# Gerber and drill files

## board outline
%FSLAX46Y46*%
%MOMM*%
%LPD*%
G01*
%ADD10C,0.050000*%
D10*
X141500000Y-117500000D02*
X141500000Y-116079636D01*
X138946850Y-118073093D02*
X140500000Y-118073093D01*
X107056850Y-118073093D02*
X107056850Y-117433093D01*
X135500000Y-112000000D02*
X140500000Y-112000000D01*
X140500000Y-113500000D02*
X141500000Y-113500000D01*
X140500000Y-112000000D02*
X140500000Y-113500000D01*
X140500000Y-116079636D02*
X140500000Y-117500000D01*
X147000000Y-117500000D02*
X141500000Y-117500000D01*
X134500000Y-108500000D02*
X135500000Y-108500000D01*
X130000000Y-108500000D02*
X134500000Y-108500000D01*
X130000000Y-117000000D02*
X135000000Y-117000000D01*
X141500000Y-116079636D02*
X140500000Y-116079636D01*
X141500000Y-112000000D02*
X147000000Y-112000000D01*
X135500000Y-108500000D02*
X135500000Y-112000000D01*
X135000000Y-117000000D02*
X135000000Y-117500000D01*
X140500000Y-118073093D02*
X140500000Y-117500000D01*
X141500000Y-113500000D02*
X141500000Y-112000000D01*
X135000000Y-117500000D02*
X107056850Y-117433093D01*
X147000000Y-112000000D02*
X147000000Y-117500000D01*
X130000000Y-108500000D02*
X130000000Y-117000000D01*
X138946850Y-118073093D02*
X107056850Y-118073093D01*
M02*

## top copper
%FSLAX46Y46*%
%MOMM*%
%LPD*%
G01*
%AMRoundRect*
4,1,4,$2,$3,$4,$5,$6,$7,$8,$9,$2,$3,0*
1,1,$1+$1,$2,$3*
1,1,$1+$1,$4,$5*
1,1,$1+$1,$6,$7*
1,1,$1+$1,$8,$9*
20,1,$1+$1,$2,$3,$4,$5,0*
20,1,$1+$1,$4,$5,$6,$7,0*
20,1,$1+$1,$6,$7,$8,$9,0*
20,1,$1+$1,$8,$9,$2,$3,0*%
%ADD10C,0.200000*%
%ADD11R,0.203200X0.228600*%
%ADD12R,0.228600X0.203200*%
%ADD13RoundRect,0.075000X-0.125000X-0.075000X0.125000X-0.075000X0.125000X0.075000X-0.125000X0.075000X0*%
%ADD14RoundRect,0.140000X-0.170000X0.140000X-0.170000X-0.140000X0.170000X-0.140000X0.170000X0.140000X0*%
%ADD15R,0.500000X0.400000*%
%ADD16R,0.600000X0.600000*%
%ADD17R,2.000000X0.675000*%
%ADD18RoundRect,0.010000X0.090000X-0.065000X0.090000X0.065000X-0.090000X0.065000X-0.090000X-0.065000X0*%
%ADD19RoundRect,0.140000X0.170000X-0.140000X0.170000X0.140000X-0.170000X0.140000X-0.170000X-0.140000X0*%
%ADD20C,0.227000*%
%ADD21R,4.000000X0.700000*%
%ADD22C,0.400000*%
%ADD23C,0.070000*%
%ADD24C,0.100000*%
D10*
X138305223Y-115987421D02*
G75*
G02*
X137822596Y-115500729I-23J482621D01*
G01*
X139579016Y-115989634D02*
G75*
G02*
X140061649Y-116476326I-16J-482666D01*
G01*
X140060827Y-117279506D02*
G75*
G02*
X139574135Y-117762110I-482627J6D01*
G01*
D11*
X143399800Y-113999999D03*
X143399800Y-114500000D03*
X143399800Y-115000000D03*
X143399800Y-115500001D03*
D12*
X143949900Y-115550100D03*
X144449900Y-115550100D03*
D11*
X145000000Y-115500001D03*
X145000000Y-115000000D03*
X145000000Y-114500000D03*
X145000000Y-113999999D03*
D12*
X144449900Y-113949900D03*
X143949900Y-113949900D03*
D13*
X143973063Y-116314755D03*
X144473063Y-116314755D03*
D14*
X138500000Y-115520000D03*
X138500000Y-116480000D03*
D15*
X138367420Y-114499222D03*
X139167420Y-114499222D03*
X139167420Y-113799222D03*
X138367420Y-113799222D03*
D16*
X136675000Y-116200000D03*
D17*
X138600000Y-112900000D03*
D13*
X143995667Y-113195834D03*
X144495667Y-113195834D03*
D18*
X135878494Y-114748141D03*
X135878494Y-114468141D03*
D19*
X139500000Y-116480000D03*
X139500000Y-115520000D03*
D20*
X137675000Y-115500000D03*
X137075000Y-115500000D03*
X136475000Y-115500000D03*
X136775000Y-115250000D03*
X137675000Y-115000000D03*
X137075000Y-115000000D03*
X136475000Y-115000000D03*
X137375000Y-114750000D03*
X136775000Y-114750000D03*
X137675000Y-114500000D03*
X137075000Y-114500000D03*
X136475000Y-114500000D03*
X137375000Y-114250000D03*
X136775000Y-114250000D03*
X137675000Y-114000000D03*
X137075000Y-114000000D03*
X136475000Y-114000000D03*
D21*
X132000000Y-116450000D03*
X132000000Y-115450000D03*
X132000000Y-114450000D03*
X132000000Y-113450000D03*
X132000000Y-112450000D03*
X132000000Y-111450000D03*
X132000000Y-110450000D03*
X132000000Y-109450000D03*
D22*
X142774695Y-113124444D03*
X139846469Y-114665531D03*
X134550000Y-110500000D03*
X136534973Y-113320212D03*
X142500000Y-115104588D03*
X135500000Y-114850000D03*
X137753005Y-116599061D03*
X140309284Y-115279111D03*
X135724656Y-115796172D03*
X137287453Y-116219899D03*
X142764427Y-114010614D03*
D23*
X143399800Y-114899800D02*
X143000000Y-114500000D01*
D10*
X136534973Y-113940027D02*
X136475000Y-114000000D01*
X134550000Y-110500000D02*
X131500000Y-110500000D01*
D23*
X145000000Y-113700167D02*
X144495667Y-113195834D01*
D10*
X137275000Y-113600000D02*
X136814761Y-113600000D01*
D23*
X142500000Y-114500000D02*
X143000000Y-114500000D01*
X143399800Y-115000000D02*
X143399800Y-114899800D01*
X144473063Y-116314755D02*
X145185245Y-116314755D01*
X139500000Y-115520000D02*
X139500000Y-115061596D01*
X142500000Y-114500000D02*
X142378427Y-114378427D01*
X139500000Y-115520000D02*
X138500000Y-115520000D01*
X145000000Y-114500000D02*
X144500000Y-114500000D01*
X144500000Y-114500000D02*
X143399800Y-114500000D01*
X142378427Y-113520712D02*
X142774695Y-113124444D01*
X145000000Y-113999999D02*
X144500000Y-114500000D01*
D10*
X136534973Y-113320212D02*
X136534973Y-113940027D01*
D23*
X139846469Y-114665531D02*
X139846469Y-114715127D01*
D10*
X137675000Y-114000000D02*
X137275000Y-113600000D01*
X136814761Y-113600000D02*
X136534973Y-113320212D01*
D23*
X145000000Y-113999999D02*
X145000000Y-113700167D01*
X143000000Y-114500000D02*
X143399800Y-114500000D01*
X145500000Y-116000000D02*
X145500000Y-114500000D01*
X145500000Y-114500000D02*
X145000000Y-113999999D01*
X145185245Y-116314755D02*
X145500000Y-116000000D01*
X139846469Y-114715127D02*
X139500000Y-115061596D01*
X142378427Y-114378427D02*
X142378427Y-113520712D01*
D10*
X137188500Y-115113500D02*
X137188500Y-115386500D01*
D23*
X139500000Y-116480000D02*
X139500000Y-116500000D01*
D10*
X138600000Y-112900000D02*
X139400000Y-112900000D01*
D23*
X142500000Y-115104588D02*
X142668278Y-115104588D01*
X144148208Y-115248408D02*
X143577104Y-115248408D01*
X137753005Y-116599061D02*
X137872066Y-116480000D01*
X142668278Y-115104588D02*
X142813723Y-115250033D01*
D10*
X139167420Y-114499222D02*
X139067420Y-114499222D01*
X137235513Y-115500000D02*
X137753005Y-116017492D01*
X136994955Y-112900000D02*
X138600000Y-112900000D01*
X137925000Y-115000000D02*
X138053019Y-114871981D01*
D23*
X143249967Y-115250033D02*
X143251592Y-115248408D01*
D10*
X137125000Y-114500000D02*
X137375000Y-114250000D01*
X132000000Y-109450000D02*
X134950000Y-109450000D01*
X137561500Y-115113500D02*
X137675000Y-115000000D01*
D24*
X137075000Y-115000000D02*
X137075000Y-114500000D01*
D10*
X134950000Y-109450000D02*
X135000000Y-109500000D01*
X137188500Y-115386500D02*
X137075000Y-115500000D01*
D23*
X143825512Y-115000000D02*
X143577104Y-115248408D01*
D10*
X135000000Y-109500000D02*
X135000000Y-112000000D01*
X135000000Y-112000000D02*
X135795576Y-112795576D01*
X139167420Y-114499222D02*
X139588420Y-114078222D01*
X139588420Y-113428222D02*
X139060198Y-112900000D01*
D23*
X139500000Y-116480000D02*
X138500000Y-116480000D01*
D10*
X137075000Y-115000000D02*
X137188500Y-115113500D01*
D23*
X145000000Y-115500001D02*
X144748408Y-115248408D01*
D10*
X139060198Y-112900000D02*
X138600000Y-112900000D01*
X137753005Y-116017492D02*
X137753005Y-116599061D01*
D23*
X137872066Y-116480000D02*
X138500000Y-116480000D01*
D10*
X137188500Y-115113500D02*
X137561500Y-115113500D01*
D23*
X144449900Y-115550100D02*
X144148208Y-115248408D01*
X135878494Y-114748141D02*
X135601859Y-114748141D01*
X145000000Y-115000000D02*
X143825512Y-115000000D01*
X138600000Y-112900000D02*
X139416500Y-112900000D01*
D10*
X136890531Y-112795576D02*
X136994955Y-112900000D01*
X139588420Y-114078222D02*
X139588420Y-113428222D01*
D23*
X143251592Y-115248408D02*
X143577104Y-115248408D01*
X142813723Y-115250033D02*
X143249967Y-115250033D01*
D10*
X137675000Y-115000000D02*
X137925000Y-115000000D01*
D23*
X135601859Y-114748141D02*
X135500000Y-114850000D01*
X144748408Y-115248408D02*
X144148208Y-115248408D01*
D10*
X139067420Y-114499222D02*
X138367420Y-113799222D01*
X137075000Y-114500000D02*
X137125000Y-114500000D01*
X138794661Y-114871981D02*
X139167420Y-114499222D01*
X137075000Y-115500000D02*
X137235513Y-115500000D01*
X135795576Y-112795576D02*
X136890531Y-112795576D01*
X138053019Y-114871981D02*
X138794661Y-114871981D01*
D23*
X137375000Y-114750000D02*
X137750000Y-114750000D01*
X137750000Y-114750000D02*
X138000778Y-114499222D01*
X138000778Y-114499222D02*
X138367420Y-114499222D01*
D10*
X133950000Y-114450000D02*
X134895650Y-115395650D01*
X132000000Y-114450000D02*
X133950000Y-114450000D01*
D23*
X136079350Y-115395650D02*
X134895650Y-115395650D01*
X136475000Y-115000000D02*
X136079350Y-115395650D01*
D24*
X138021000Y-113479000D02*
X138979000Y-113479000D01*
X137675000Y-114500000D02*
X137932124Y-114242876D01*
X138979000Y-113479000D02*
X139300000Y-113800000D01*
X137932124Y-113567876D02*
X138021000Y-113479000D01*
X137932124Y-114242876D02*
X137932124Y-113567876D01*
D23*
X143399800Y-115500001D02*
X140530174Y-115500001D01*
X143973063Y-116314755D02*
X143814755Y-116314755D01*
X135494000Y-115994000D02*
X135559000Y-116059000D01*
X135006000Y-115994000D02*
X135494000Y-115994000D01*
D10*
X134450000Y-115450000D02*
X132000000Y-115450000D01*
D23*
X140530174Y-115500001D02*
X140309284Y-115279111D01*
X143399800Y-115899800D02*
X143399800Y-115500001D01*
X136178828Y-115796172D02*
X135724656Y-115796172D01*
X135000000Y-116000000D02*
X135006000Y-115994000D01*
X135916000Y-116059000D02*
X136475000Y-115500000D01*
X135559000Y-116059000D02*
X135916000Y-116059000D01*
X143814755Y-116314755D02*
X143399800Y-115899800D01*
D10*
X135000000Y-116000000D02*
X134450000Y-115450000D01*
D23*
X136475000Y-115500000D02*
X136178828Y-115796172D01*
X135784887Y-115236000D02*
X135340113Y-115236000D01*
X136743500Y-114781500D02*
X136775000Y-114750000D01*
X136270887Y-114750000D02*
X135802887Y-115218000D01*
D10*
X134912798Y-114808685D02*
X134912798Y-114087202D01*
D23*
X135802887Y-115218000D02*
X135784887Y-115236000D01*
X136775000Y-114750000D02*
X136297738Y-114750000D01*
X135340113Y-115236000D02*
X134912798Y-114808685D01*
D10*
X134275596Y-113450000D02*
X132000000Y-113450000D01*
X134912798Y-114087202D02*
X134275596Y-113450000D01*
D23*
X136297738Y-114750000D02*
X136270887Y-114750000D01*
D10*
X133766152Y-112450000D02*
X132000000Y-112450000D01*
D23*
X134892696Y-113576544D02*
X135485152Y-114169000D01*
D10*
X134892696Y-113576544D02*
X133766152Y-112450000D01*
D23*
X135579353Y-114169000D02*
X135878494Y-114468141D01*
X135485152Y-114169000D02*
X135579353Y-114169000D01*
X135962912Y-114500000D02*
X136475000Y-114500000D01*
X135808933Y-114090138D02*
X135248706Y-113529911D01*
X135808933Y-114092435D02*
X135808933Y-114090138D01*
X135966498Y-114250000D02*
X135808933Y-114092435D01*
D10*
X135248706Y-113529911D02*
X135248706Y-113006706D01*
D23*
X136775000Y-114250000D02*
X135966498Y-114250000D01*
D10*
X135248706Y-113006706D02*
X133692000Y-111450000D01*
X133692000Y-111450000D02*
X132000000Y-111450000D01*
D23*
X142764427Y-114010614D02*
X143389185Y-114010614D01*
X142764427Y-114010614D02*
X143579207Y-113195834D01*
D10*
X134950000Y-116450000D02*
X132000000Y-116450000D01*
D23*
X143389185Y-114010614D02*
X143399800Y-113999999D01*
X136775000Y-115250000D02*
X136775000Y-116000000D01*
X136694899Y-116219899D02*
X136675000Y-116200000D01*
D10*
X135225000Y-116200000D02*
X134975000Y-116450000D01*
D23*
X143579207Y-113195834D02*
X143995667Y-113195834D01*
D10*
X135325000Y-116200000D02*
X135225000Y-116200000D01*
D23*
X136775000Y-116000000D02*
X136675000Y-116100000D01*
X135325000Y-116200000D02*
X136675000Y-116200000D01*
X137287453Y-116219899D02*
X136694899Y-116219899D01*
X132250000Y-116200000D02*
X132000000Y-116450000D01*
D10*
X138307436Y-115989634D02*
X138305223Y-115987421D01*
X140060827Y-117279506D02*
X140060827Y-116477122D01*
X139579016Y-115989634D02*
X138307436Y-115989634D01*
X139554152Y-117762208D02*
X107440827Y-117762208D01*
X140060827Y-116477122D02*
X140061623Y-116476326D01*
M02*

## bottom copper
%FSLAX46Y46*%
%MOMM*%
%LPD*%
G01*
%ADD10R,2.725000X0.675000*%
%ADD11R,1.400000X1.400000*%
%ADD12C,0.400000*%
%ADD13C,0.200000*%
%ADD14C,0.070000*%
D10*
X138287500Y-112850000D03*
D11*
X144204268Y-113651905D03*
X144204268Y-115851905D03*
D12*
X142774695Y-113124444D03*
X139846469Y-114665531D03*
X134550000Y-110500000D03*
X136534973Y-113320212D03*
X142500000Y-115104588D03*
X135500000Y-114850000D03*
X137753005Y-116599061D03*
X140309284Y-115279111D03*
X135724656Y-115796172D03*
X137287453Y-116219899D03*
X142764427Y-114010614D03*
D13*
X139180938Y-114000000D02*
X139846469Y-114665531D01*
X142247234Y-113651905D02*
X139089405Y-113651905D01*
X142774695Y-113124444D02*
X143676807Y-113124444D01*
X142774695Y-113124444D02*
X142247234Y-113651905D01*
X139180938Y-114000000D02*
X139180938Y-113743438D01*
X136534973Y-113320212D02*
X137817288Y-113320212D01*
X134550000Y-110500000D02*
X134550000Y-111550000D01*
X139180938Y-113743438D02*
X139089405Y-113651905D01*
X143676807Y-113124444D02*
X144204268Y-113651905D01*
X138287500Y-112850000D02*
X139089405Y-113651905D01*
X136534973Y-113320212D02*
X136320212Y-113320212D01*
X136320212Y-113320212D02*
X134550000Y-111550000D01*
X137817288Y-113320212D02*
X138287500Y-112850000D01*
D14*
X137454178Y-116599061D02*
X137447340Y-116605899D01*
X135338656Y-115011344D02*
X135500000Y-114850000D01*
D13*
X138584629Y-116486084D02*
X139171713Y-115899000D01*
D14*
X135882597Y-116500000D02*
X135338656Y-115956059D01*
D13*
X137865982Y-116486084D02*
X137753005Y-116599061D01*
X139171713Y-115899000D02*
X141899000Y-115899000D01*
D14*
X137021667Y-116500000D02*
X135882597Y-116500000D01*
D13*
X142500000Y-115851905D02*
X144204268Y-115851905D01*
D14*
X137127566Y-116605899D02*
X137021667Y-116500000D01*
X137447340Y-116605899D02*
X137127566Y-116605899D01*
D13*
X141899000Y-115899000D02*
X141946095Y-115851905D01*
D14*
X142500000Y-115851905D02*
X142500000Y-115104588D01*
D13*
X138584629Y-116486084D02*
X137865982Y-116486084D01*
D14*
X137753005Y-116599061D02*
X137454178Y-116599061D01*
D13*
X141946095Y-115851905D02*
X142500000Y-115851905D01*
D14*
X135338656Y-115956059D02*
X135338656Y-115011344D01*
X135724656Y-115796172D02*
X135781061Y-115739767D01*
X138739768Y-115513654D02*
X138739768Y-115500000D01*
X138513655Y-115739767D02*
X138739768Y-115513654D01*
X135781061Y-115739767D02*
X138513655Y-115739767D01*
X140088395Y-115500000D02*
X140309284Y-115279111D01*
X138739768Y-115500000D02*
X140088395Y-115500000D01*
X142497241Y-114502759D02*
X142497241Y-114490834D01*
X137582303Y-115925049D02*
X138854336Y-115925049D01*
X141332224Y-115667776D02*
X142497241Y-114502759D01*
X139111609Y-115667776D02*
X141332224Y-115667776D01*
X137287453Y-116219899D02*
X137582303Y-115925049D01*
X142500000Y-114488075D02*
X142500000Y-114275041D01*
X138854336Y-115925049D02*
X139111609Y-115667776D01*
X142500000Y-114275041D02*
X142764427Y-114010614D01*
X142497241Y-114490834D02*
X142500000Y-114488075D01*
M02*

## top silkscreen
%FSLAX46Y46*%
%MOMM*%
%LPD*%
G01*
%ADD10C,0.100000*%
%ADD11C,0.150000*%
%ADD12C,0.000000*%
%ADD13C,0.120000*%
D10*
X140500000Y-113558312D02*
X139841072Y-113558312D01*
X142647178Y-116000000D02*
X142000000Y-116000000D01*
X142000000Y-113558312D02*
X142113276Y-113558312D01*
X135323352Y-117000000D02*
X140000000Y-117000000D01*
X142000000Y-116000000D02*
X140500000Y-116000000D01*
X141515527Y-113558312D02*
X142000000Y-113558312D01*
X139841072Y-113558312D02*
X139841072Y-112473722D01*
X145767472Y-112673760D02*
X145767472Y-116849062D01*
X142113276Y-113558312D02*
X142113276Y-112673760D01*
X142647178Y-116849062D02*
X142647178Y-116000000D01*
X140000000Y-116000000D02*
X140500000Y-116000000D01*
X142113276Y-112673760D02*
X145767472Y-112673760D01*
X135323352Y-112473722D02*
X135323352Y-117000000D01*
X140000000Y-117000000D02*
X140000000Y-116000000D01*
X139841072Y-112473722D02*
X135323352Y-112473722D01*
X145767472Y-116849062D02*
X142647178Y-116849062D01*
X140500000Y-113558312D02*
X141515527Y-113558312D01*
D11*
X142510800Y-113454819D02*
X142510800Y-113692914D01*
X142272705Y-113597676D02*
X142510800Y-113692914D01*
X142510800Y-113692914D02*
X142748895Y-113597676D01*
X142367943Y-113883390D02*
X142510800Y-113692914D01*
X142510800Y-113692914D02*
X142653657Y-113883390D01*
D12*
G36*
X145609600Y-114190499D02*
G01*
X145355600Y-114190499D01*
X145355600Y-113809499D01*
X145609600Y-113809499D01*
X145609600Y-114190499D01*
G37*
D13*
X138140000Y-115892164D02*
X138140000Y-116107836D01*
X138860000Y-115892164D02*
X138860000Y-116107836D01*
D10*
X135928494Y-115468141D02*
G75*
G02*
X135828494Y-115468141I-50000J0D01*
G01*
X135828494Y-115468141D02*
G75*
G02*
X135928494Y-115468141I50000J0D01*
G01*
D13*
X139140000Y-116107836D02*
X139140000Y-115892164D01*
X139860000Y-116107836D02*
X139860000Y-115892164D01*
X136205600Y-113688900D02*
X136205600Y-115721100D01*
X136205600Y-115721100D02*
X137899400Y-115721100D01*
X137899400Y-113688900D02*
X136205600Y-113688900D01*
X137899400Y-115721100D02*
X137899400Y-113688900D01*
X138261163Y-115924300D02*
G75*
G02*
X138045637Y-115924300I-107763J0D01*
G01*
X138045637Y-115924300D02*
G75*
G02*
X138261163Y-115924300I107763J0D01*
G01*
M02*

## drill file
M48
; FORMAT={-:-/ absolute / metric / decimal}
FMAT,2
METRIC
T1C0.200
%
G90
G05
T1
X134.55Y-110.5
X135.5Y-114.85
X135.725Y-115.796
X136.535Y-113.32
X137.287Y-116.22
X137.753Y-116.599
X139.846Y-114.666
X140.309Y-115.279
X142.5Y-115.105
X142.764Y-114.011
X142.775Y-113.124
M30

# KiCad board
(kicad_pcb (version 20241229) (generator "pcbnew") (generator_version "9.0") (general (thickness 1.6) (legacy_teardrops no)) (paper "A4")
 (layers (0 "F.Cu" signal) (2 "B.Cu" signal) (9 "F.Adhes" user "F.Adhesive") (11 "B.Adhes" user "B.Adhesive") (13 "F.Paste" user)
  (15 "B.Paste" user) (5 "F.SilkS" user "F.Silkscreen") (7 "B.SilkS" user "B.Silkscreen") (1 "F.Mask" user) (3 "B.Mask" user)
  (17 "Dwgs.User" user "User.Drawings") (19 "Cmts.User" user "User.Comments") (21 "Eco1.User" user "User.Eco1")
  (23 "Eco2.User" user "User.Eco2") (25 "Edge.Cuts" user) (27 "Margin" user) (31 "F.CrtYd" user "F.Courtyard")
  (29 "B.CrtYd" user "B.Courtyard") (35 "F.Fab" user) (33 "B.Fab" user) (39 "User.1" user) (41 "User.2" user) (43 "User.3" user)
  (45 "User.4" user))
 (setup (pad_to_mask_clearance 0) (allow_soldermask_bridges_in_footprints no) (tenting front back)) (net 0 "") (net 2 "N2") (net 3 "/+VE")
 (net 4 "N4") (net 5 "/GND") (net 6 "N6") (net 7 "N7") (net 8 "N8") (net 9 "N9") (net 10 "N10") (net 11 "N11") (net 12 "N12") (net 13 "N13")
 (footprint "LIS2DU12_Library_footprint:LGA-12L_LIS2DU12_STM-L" (layer "F.Cu") (at 144.1999 114.75)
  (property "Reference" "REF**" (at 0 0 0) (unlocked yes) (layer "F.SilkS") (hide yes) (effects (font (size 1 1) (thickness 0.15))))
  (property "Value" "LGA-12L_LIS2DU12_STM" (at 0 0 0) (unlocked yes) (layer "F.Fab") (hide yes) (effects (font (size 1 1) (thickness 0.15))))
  (fp_poly
   (pts (xy 1.4097 -0.940501) (xy 1.4097 -0.559501) (xy 1.1557 -0.559501) (xy 1.1557 -0.940501)) (stroke (width 0) (type solid)) (fill yes)
   (layer "F.SilkS") (net 1))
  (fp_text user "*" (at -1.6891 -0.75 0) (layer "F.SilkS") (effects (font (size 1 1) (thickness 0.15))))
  (pad "1" smd rect (at -0.8001 -0.750001 90) (size 0.2286 0.2032) (layers "F.Cu" "F.Mask" "F.Paste") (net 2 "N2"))
  (pad "2" smd rect (at -0.8001 -0.25 90) (size 0.2286 0.2032) (layers "F.Cu" "F.Mask" "F.Paste") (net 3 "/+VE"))
  (pad "3" smd rect (at -0.8001 0.25 90) (size 0.2286 0.2032) (layers "F.Cu" "F.Mask" "F.Paste") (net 3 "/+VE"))
  (pad "4" smd rect (at -0.8001 0.750001 90) (size 0.2286 0.2032) (layers "F.Cu" "F.Mask" "F.Paste") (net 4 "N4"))
  (pad "5" smd rect (at -0.25 0.8001) (size 0.2286 0.2032) (layers "F.Cu" "F.Mask" "F.Paste"))
  (pad "6" smd rect (at 0.25 0.8001) (size 0.2286 0.2032) (layers "F.Cu" "F.Mask" "F.Paste") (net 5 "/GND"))
  (pad "7" smd rect (at 0.8001 0.750001 90) (size 0.2286 0.2032) (layers "F.Cu" "F.Mask" "F.Paste") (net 5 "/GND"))
  (pad "8" smd rect (at 0.8001 0.25 90) (size 0.2286 0.2032) (layers "F.Cu" "F.Mask" "B.Adhes" "F.Paste") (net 5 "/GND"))
  (pad "9" smd rect (at 0.8001 -0.25 90) (size 0.2286 0.2032) (layers "F.Cu" "F.Mask" "F.Paste") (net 3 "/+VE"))
  (pad "10" smd rect (at 0.8001 -0.750001 90) (size 0.2286 0.2032) (layers "F.Cu" "F.Mask" "F.Paste") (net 3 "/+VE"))
  (pad "11" smd rect (at 0.25 -0.8001) (size 0.2286 0.2032) (layers "F.Cu" "F.Mask" "F.Paste"))
  (pad "12" smd rect (at -0.25 -0.8001) (size 0.2286 0.2032) (layers "F.Cu" "F.Mask" "F.Paste")))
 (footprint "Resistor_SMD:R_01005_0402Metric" (layer "F.Cu") (at 144.223063 116.314755)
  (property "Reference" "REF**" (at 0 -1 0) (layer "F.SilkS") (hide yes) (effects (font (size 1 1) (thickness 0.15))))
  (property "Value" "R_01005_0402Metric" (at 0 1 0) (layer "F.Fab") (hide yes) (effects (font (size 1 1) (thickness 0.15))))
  (pad "" smd roundrect (at -0.275 0) (size 0.27 0.27) (layers "F.Paste") (roundrect_rratio 0.25))
  (pad "" smd roundrect (at 0.275 0) (size 0.27 0.27) (layers "F.Paste") (roundrect_rratio 0.25))
  (pad "1" smd roundrect (at -0.25 0) (size 0.4 0.3) (layers "F.Cu" "F.Mask") (roundrect_rratio 0.25) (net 4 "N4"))
  (pad "2" smd roundrect (at 0.25 0) (size 0.4 0.3) (layers "F.Cu" "F.Mask") (roundrect_rratio 0.25) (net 3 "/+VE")))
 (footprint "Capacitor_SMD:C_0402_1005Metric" (layer "F.Cu") (at 138.5 116 -90)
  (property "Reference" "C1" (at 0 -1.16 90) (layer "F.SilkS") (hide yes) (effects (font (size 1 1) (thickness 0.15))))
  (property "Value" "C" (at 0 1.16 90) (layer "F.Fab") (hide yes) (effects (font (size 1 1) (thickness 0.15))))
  (fp_line (start -0.107836 0.36) (end 0.107836 0.36) (stroke (width 0.12) (type solid)) (layer "F.SilkS") (net 1))
  (fp_line (start -0.107836 -0.36) (end 0.107836 -0.36) (stroke (width 0.12) (type solid)) (layer "F.SilkS") (net 1))
  (pad "1" smd roundrect (at -0.48 0 270) (size 0.56 0.62) (layers "F.Cu" "F.Mask" "F.Paste") (roundrect_rratio 0.25) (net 3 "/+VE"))
  (pad "2" smd roundrect (at 0.48 0 270) (size 0.56 0.62) (layers "F.Cu" "F.Mask" "F.Paste") (roundrect_rratio 0.25) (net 5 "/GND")))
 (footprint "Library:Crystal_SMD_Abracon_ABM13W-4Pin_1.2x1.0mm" (layer "F.Cu") (at 138.76742 114.149222)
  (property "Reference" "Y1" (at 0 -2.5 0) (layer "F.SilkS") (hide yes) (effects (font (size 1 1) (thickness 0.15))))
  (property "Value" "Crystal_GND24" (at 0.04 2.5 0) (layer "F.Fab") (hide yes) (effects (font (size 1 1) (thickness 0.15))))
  (pad "1" smd rect (at -0.4 0.35) (size 0.5 0.4) (layers "F.Cu" "F.Mask" "F.Paste") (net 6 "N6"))
  (pad "2" smd rect (at 0.4 0.35) (size 0.5 0.4) (layers "F.Cu" "F.Mask" "F.Paste") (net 5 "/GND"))
  (pad "3" smd rect (at 0.4 -0.35) (size 0.5 0.4) (layers "F.Cu" "F.Mask" "F.Paste") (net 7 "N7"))
  (pad "4" smd rect (at -0.4 -0.35) (size 0.5 0.4) (layers "F.Cu" "F.Mask" "F.Paste") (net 5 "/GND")))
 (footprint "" (layer "F.Cu") (at 137.075 115.9 180)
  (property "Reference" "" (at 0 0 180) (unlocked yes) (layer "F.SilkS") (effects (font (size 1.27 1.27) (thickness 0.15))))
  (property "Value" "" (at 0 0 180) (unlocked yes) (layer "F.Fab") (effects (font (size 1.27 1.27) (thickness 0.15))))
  (pad "2" smd rect (at 0.4 -0.3 90) (size 0.6 0.6) (layers "F.Cu" "F.Mask" "F.Paste") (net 2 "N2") (solder_mask_margin 0.102)))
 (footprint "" (layer "F.Cu") (at 138.5 113)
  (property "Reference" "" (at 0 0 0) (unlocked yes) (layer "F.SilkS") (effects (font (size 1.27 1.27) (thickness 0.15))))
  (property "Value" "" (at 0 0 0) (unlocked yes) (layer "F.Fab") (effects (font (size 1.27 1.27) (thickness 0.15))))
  (pad "2" smd rect (at 0.1 -0.1 270) (size 0.675 2) (layers "F.Cu" "F.Mask" "F.Paste") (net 5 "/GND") (solder_mask_margin 0.102)))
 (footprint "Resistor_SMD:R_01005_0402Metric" (layer "F.Cu") (at 144.245667 113.195834)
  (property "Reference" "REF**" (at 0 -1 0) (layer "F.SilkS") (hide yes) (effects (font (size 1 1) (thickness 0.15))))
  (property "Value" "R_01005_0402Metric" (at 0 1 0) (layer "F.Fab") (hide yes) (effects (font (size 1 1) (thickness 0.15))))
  (pad "" smd roundrect (at -0.275 0) (size 0.27 0.27) (layers "F.Paste") (roundrect_rratio 0.25))
  (pad "" smd roundrect (at 0.275 0) (size 0.27 0.27) (layers "F.Paste") (roundrect_rratio 0.25))
  (pad "1" smd roundrect (at -0.25 0) (size 0.4 0.3) (layers "F.Cu" "F.Mask") (roundrect_rratio 0.25) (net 2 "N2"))
  (pad "2" smd roundrect (at 0.25 0) (size 0.4 0.3) (layers "F.Cu" "F.Mask") (roundrect_rratio 0.25) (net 3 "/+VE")))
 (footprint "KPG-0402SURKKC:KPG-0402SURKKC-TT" (layer "F.Cu") (at 135.878494 114.608141 90)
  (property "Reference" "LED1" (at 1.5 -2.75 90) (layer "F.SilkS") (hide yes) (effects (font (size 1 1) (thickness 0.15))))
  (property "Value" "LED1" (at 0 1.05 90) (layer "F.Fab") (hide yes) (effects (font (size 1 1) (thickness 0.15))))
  (fp_circle (center -0.86 0) (end -0.81 0) (stroke (width 0.1) (type solid)) (fill no) (layer "F.SilkS") (net 1))
  (pad "" smd roundrect (at -0.14 0 90) (size 0.15 0.2) (layers "F.Mask") (roundrect_rratio 0.06666666667))
  (pad "" smd roundrect (at -0.1225 0 90) (size 0.1 0.17) (layers "F.Paste") (roundrect_rratio 0.25))
  (pad "" smd roundrect (at 0.1225 0 90) (size 0.1 0.17) (layers "F.Paste") (roundrect_rratio 0.25))
  (pad "" smd roundrect (at 0.14 0 90) (size 0.15 0.2) (layers "F.Mask") (roundrect_rratio 0.06666666667))
  (pad "1" smd roundrect (at -0.14 0 90) (size 0.15 0.2) (layers "F.Cu" "F.Mask") (roundrect_rratio 0.06666666667) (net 5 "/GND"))
  (pad "2" smd roundrect (at 0.14 0 90) (size 0.15 0.2) (layers "F.Cu" "F.Mask") (roundrect_rratio 0.06666666667) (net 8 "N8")))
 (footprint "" (layer "F.Cu") (at 138.4 112.5875 180)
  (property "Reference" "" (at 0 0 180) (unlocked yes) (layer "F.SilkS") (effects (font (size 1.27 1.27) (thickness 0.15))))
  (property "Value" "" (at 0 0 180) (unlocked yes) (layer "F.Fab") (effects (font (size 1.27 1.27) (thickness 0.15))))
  (pad "2" smd rect (at 0.1125 -0.2625 90) (size 0.675 2.725) (layers "B.Cu" "B.Mask" "B.Paste") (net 3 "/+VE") (solder_mask_margin 0.102)))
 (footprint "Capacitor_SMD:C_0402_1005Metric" (layer "F.Cu") (at 139.5 116 90)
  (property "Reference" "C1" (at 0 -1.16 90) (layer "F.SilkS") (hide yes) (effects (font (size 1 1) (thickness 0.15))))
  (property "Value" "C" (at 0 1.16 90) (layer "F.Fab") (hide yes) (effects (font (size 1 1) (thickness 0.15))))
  (fp_line (start -0.107836 -0.36) (end 0.107836 -0.36) (stroke (width 0.12) (type solid)) (layer "F.SilkS") (net 1))
  (fp_line (start -0.107836 0.36) (end 0.107836 0.36) (stroke (width 0.12) (type solid)) (layer "F.SilkS") (net 1))
  (pad "1" smd roundrect (at -0.48 0 90) (size 0.56 0.62) (layers "F.Cu" "F.Mask" "F.Paste") (roundrect_rratio 0.25) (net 5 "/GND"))
  (pad "2" smd roundrect (at 0.48 0 90) (size 0.56 0.62) (layers "F.Cu" "F.Mask" "F.Paste") (roundrect_rratio 0.25) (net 3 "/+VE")))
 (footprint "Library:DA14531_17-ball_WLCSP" (layer "F.Cu") (at 137.053 114.705 180)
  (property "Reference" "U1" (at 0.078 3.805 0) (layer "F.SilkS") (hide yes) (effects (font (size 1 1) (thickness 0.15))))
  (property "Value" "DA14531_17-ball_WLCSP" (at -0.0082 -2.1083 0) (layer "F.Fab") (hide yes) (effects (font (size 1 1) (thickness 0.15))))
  (fp_line (start 0.8474 1.0161) (end 0.8474 -1.0161) (stroke (width 0.12) (type solid)) (layer "F.SilkS") (net 1))
  (fp_line (start 0.8474 -1.0161) (end -0.8464 -1.0161) (stroke (width 0.12) (type solid)) (layer "F.SilkS") (net 1))
  (fp_line (start -0.8464 1.0161) (end 0.8474 1.0161) (stroke (width 0.12) (type solid)) (layer "F.SilkS") (net 1))
  (fp_line (start -0.8464 -1.0161) (end -0.8464 1.0161) (stroke (width 0.12) (type solid)) (layer "F.SilkS") (net 1))
  (fp_circle (center -1.1004 -1.2193) (end -1.0242 -1.1431) (stroke (width 0.12) (type solid)) (fill no) (layer "F.SilkS") (net 1))
  (pad "A1" smd circle (at -0.622 -0.795 180) (size 0.227 0.227) (layers "F.Cu" "F.Mask" "F.Paste") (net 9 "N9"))
  (pad "A3" smd circle (at -0.022 -0.795 180) (size 0.227 0.227) (layers "F.Cu" "F.Mask" "F.Paste") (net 5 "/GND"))
  (pad "A5" smd circle (at 0.578 -0.795 180) (size 0.227 0.227) (layers "F.Cu" "F.Mask" "F.Paste") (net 4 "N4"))
  (pad "B4" smd circle (at 0.278 -0.545 180) (size 0.227 0.227) (layers "F.Cu" "F.Mask" "F.Paste") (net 2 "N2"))
  (pad "C1" smd circle (at -0.622 -0.295 180) (size 0.227 0.227) (layers "F.Cu" "F.Mask" "F.Paste") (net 5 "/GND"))
  (pad "C3" smd circle (at -0.022 -0.295 180) (size 0.227 0.227) (layers "F.Cu" "F.Mask" "F.Paste") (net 5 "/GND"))
  (pad "C5" smd circle (at 0.578 -0.295 180) (size 0.227 0.227) (layers "F.Cu" "F.Mask" "F.Paste") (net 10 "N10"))
  (pad "D2" smd circle (at -0.322 -0.045 180) (size 0.227 0.227) (layers "F.Cu" "F.Mask" "F.Paste") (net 6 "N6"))
  (pad "D4" smd circle (at 0.278 -0.045 180) (size 0.227 0.227) (layers "F.Cu" "F.Mask" "F.Paste") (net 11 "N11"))
  (pad "E1" smd circle (at -0.622 0.205 180) (size 0.227 0.227) (layers "F.Cu" "F.Mask" "F.Paste") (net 7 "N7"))
  (pad "E3" smd circle (at -0.022 0.205 180) (size 0.227 0.227) (layers "F.Cu" "F.Mask" "F.Paste") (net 5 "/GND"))
  (pad "E5" smd circle (at 0.578 0.205 180) (size 0.227 0.227) (layers "F.Cu" "F.Mask" "F.Paste") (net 8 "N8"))
  (pad "F2" smd circle (at -0.322 0.455 180) (size 0.227 0.227) (layers "F.Cu" "F.Mask" "F.Paste") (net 5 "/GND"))
  (pad "F4" smd circle (at 0.278 0.455 180) (size 0.227 0.227) (layers "F.Cu" "F.Mask" "F.Paste") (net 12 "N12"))
  (pad "G1" smd circle (at -0.622 0.705 180) (size 0.227 0.227) (layers "F.Cu" "F.Mask" "F.Paste") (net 3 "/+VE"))
  (pad "G3" smd circle (at -0.022 0.705 180) (size 0.227 0.227) (layers "F.Cu" "F.Mask" "F.Paste") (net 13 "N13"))
  (pad "G5" smd circle (at 0.578 0.705 180) (size 0.227 0.227) (layers "F.Cu" "F.Mask" "F.Paste") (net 3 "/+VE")))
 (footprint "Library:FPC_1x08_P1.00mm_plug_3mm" (layer "F.Cu") (at 134 112.95 180)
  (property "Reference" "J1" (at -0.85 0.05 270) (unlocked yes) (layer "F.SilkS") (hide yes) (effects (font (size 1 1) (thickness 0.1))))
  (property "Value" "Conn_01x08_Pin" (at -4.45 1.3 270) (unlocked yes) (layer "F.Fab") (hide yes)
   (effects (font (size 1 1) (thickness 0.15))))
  (pad "1" connect rect (at 2 -3.5 180) (size 4 0.7) (layers "F.Cu" "F.Mask") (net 2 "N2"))
  (pad "2" connect rect (at 2 -2.5 180) (size 4 0.7) (layers "F.Cu" "F.Mask") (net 4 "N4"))
  (pad "3" connect rect (at 2 -1.5 180) (size 4 0.7) (layers "F.Cu" "F.Mask") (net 10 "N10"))
  (pad "4" connect rect (at 2 -0.5 180) (size 4 0.7) (layers "F.Cu" "F.Mask") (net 11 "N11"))
  (pad "5" connect rect (at 2 0.5 180) (size 4 0.7) (layers "F.Cu" "F.Mask") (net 8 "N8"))
  (pad "6" connect rect (at 2 1.5 180) (size 4 0.7) (layers "F.Cu" "F.Mask") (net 12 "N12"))
  (pad "7" connect rect (at 2 2.5 180) (size 4 0.7) (layers "F.Cu" "F.Mask") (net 3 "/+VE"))
  (pad "8" connect rect (at 2 3.5 180) (size 4 0.7) (layers "F.Cu" "F.Mask") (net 5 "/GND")))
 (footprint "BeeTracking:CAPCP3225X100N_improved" (layer "B.Cu") (at 144.204268 114.751905 -90)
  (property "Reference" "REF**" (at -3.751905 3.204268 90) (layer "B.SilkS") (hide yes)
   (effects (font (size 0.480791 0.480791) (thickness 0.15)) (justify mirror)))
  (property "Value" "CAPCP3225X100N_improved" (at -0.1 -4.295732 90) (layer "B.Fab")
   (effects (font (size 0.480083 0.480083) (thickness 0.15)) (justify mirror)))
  (pad "1" smd rect (at -1.1 0 90) (size 1.4 1.4) (layers "B.Cu" "B.Mask" "B.Paste") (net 3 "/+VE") (solder_mask_margin 0.102))
  (pad "2" smd rect (at 1.1 0 90) (size 1.4 1.4) (layers "B.Cu" "B.Mask" "B.Paste") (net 5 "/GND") (solder_mask_margin 0.102)))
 (gr_arc (start 138.305223 115.987421) (mid 137.962521 115.844622) (end 137.822616 115.500729) (stroke (width 0.2) (type default))
  (layer "F.Cu") (net 9))
 (gr_arc (start 139.579016 115.989634) (mid 139.921718 116.132433) (end 140.061623 116.476326) (stroke (width 0.2) (type default))
  (layer "F.Cu") (net 9))
 (gr_arc (start 140.060827 117.279506) (mid 139.918028 117.622208) (end 139.574135 117.762113) (stroke (width 0.2) (type default))
  (layer "F.Cu") (net 9))
 (gr_line (start 140.5 113.558312) (end 139.841072 113.558312) (stroke (width 0.1) (type default)) (layer "F.SilkS"))
 (gr_line (start 142.647178 116) (end 142 116) (stroke (width 0.1) (type default)) (layer "F.SilkS"))
 (gr_line (start 142 113.558312) (end 142.113276 113.558312) (stroke (width 0.1) (type default)) (layer "F.SilkS"))
 (gr_line (start 135.323352 117) (end 140 117) (stroke (width 0.1) (type default)) (layer "F.SilkS"))
 (gr_line (start 142 116) (end 140.5 116) (stroke (width 0.1) (type default)) (layer "F.SilkS"))
 (gr_line (start 141.515527 113.558312) (end 142 113.558312) (stroke (width 0.1) (type default)) (layer "F.SilkS"))
 (gr_line (start 139.841072 113.558312) (end 139.841072 112.473722) (stroke (width 0.1) (type default)) (layer "F.SilkS"))
 (gr_line (start 145.767472 112.67376) (end 145.767472 116.849062) (stroke (width 0.1) (type default)) (layer "F.SilkS"))
 (gr_line (start 142.113276 113.558312) (end 142.113276 112.67376) (stroke (width 0.1) (type default)) (layer "F.SilkS"))
 (gr_line (start 142.647178 116.849062) (end 142.647178 116) (stroke (width 0.1) (type default)) (layer "F.SilkS"))
 (gr_line (start 140 116) (end 140.5 116) (stroke (width 0.1) (type default)) (layer "F.SilkS"))
 (gr_line (start 142.113276 112.67376) (end 145.767472 112.67376) (stroke (width 0.1) (type default)) (layer "F.SilkS"))
 (gr_line (start 135.323352 112.473722) (end 135.323352 117) (stroke (width 0.1) (type default)) (layer "F.SilkS"))
 (gr_line (start 140 117) (end 140 116) (stroke (width 0.1) (type default)) (layer "F.SilkS"))
 (gr_line (start 139.841072 112.473722) (end 135.323352 112.473722) (stroke (width 0.1) (type default)) (layer "F.SilkS"))
 (gr_line (start 145.767472 116.849062) (end 142.647178 116.849062) (stroke (width 0.1) (type default)) (layer "F.SilkS"))
 (gr_line (start 140.5 113.558312) (end 141.515527 113.558312) (stroke (width 0.1) (type default)) (layer "F.SilkS"))
 (gr_line (start 141.5 117.5) (end 141.5 116.079636) (stroke (width 0.05) (type default)) (layer "Edge.Cuts"))
 (gr_line (start 138.94685 118.073093) (end 140.5 118.073093) (stroke (width 0.05) (type default)) (layer "Edge.Cuts"))
 (gr_line (start 107.05685 118.073093) (end 107.05685 117.433093) (stroke (width 0.05) (type default)) (layer "Edge.Cuts"))
 (gr_line (start 135.5 112) (end 140.5 112) (stroke (width 0.05) (type default)) (layer "Edge.Cuts"))
 (gr_line (start 140.5 113.5) (end 141.5 113.5) (stroke (width 0.05) (type default)) (layer "Edge.Cuts"))
 (gr_line (start 140.5 112) (end 140.5 113.5) (stroke (width 0.05) (type default)) (layer "Edge.Cuts"))
 (gr_line (start 140.5 116.079636) (end 140.5 117.5) (stroke (width 0.05) (type default)) (layer "Edge.Cuts"))
 (gr_line (start 147 117.5) (end 141.5 117.5) (stroke (width 0.05) (type default)) (layer "Edge.Cuts"))
 (gr_line (start 134.5 108.5) (end 135.5 108.5) (stroke (width 0.05) (type default)) (layer "Edge.Cuts"))
 (gr_line (start 130 108.5) (end 134.5 108.5) (stroke (width 0.05) (type default)) (layer "Edge.Cuts"))
 (gr_line (start 130 117) (end 135 117) (stroke (width 0.05) (type default)) (layer "Edge.Cuts"))
 (gr_line (start 141.5 116.079636) (end 140.5 116.079636) (stroke (width 0.05) (type default)) (layer "Edge.Cuts"))
 (gr_line (start 141.5 112) (end 147 112) (stroke (width 0.05) (type default)) (layer "Edge.Cuts"))
 (gr_line (start 135.5 108.5) (end 135.5 112) (stroke (width 0.05) (type default)) (layer "Edge.Cuts"))
 (gr_line (start 135 117) (end 135 117.5) (stroke (width 0.05) (type default)) (layer "Edge.Cuts"))
 (gr_line (start 140.5 118.073093) (end 140.5 117.5) (stroke (width 0.05) (type default)) (layer "Edge.Cuts"))
 (gr_line (start 141.5 113.5) (end 141.5 112) (stroke (width 0.05) (type default)) (layer "Edge.Cuts"))
 (gr_line (start 135 117.5) (end 107.05685 117.433093) (stroke (width 0.05) (type default)) (layer "Edge.Cuts"))
 (gr_line (start 147 112) (end 147 117.5) (stroke (width 0.05) (type default)) (layer "Edge.Cuts"))
 (gr_line (start 130 108.5) (end 130 117) (stroke (width 0.05) (type default)) (layer "Edge.Cuts"))
 (gr_line (start 138.94685 118.073093) (end 107.05685 118.073093) (stroke (width 0.05) (type default)) (layer "Edge.Cuts"))
 (segment (start 143.3998 114.8998) (end 143 114.5) (width 0.07) (layer "F.Cu") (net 3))
 (segment (start 136.534973 113.940027) (end 136.475 114) (width 0.2) (layer "F.Cu") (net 3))
 (segment (start 134.55 110.5) (end 131.5 110.5) (width 0.2) (layer "F.Cu") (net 3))
 (segment (start 145 113.700167) (end 144.495667 113.195834) (width 0.07) (layer "F.Cu") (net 3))
 (segment (start 137.275 113.6) (end 136.814761 113.6) (width 0.2) (layer "F.Cu") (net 3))
 (segment (start 142.5 114.5) (end 143 114.5) (width 0.07) (layer "F.Cu") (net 3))
 (segment (start 143.3998 115) (end 143.3998 114.8998) (width 0.07) (layer "F.Cu") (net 3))
 (segment (start 144.473063 116.314755) (end 145.185245 116.314755) (width 0.07) (layer "F.Cu") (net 3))
 (segment (start 139.5 115.52) (end 139.5 115.061596) (width 0.07) (layer "F.Cu") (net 3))
 (segment (start 142.5 114.5) (end 142.378427 114.378427) (width 0.07) (layer "F.Cu") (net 3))
 (segment (start 139.5 115.52) (end 138.5 115.52) (width 0.07) (layer "F.Cu") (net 3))
 (segment (start 145 114.5) (end 144.5 114.5) (width 0.07) (layer "F.Cu") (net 3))
 (segment (start 144.5 114.5) (end 143.3998 114.5) (width 0.07) (layer "F.Cu") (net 3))
 (segment (start 142.378427 113.520712) (end 142.774695 113.124444) (width 0.07) (layer "F.Cu") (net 3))
 (segment (start 145 113.999999) (end 144.5 114.5) (width 0.07) (layer "F.Cu") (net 3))
 (segment (start 136.534973 113.320212) (end 136.534973 113.940027) (width 0.2) (layer "F.Cu") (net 3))
 (segment (start 139.846469 114.665531) (end 139.846469 114.715127) (width 0.07) (layer "F.Cu") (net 3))
 (segment (start 137.675 114) (end 137.275 113.6) (width 0.2) (layer "F.Cu") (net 3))
 (segment (start 136.814761 113.6) (end 136.534973 113.320212) (width 0.2) (layer "F.Cu") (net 3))
 (segment (start 145 113.999999) (end 145 113.700167) (width 0.07) (layer "F.Cu") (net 3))
 (segment (start 143 114.5) (end 143.3998 114.5) (width 0.07) (layer "F.Cu") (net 3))
 (segment (start 145.5 116) (end 145.5 114.5) (width 0.07) (layer "F.Cu") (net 3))
 (segment (start 145.5 114.5) (end 145 113.999999) (width 0.07) (layer "F.Cu") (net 3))
 (segment (start 145.185245 116.314755) (end 145.5 116) (width 0.07) (layer "F.Cu") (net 3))
 (segment (start 139.846469 114.715127) (end 139.5 115.061596) (width 0.07) (layer "F.Cu") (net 3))
 (segment (start 142.378427 114.378427) (end 142.378427 113.520712) (width 0.07) (layer "F.Cu") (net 3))
 (via (at 142.774695 113.124444) (size 0.4) (drill 0.2) (layers "F.Cu" "B.Cu") (free yes) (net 3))
 (via (at 139.846469 114.665531) (size 0.4) (drill 0.2) (layers "F.Cu" "B.Cu") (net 3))
 (via (at 134.55 110.5) (size 0.4) (drill 0.2) (layers "F.Cu" "B.Cu") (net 3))
 (via (at 136.534973 113.320212) (size 0.4) (drill 0.2) (layers "F.Cu" "B.Cu") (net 3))
 (segment (start 139.180938 114) (end 139.846469 114.665531) (width 0.2) (layer "B.Cu") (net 3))
 (segment (start 142.247234 113.651905) (end 139.089405 113.651905) (width 0.2) (layer "B.Cu") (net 3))
 (segment (start 142.774695 113.124444) (end 143.676807 113.124444) (width 0.2) (layer "B.Cu") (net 3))
 (segment (start 142.774695 113.124444) (end 142.247234 113.651905) (width 0.2) (layer "B.Cu") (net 3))
 (segment (start 139.180938 114) (end 139.180938 113.743438) (width 0.2) (layer "B.Cu") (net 3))
 (segment (start 136.534973 113.320212) (end 137.817288 113.320212) (width 0.2) (layer "B.Cu") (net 3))
 (segment (start 134.55 110.5) (end 134.55 111.55) (width 0.2) (layer "B.Cu") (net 3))
 (segment (start 139.180938 113.743438) (end 139.089405 113.651905) (width 0.2) (layer "B.Cu") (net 3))
 (segment (start 143.676807 113.124444) (end 144.204268 113.651905) (width 0.2) (layer "B.Cu") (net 3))
 (segment (start 138.2875 112.85) (end 139.089405 113.651905) (width 0.2) (layer "B.Cu") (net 3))
 (segment (start 136.534973 113.320212) (end 136.320212 113.320212) (width 0.2) (layer "B.Cu") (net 3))
 (segment (start 136.320212 113.320212) (end 134.55 111.55) (width 0.2) (layer "B.Cu") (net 3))
 (segment (start 137.817288 113.320212) (end 138.2875 112.85) (width 0.2) (layer "B.Cu") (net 3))
 (segment (start 137.1885 115.1135) (end 137.1885 115.3865) (width 0.2) (layer "F.Cu") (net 5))
 (segment (start 139.5 116.48) (end 139.5 116.5) (width 0.07) (layer "F.Cu") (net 5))
 (segment (start 138.6 112.9) (end 139.4 112.9) (width 0.2) (layer "F.Cu") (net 5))
 (segment (start 142.5 115.104588) (end 142.668278 115.104588) (width 0.07) (layer "F.Cu") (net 5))
 (segment (start 144.148208 115.248408) (end 143.577104 115.248408) (width 0.07) (layer "F.Cu") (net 5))
 (segment (start 137.753005 116.599061) (end 137.872066 116.48) (width 0.07) (layer "F.Cu") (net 5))
 (segment (start 142.668278 115.104588) (end 142.813723 115.250033) (width 0.07) (layer "F.Cu") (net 5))
 (segment (start 139.16742 114.499222) (end 139.06742 114.499222) (width 0.2) (layer "F.Cu") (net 5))
 (segment (start 137.235513 115.5) (end 137.753005 116.017492) (width 0.2) (layer "F.Cu") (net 5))
 (segment (start 136.994955 112.9) (end 138.6 112.9) (width 0.2) (layer "F.Cu") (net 5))
 (segment (start 137.925 115) (end 138.053019 114.871981) (width 0.2) (layer "F.Cu") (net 5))
 (segment (start 143.249967 115.250033) (end 143.251592 115.248408) (width 0.07) (layer "F.Cu") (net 5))
 (segment (start 137.125 114.5) (end 137.375 114.25) (width 0.2) (layer "F.Cu") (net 5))
 (segment (start 132 109.45) (end 134.95 109.45) (width 0.2) (layer "F.Cu") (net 5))
 (segment (start 137.5615 115.1135) (end 137.675 115) (width 0.2) (layer "F.Cu") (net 5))
 (segment (start 137.075 115) (end 137.075 114.5) (width 0.1) (layer "F.Cu") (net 5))
 (segment (start 134.95 109.45) (end 135 109.5) (width 0.2) (layer "F.Cu") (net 5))
 (segment (start 137.1885 115.3865) (end 137.075 115.5) (width 0.2) (layer "F.Cu") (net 5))
 (segment (start 143.825512 115) (end 143.577104 115.248408) (width 0.07) (layer "F.Cu") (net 5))
 (segment (start 135 109.5) (end 135 112) (width 0.2) (layer "F.Cu") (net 5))
 (segment (start 135 112) (end 135.795576 112.795576) (width 0.2) (layer "F.Cu") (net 5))
 (segment (start 139.16742 114.499222) (end 139.58842 114.078222) (width 0.2) (layer "F.Cu") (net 5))
 (segment (start 139.58842 113.428222) (end 139.060198 112.9) (width 0.2) (layer "F.Cu") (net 5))
 (segment (start 139.5 116.48) (end 138.5 116.48) (width 0.07) (layer "F.Cu") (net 5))
 (segment (start 137.075 115) (end 137.1885 115.1135) (width 0.2) (layer "F.Cu") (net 5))
 (segment (start 145 115.500001) (end 144.748408 115.248408) (width 0.07) (layer "F.Cu") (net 5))
 (segment (start 139.060198 112.9) (end 138.6 112.9) (width 0.2) (layer "F.Cu") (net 5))
 (segment (start 137.753005 116.017492) (end 137.753005 116.599061) (width 0.2) (layer "F.Cu") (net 5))
 (segment (start 137.872066 116.48) (end 138.5 116.48) (width 0.07) (layer "F.Cu") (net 5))
 (segment (start 137.1885 115.1135) (end 137.5615 115.1135) (width 0.2) (layer "F.Cu") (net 5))
 (segment (start 144.4499 115.5501) (end 144.148208 115.248408) (width 0.07) (layer "F.Cu") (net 5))
 (segment (start 135.878494 114.748141) (end 135.601859 114.748141) (width 0.07) (layer "F.Cu") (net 5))
 (segment (start 145 115) (end 143.825512 115) (width 0.07) (layer "F.Cu") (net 5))
 (segment (start 138.6 112.9) (end 139.4165 112.9) (width 0.07) (layer "F.Cu") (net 5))
 (segment (start 136.890531 112.795576) (end 136.994955 112.9) (width 0.2) (layer "F.Cu") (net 5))
 (segment (start 139.58842 114.078222) (end 139.58842 113.428222) (width 0.2) (layer "F.Cu") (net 5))
 (segment (start 143.251592 115.248408) (end 143.577104 115.248408) (width 0.07) (layer "F.Cu") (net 5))
 (segment (start 142.813723 115.250033) (end 143.249967 115.250033) (width 0.07) (layer "F.Cu") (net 5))
 (segment (start 137.675 115) (end 137.925 115) (width 0.2) (layer "F.Cu") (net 5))
 (segment (start 135.601859 114.748141) (end 135.5 114.85) (width 0.07) (layer "F.Cu") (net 5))
 (segment (start 144.748408 115.248408) (end 144.148208 115.248408) (width 0.07) (layer "F.Cu") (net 5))
 (segment (start 139.06742 114.499222) (end 138.36742 113.799222) (width 0.2) (layer "F.Cu") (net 5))
 (segment (start 137.075 114.5) (end 137.125 114.5) (width 0.2) (layer "F.Cu") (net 5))
 (segment (start 138.794661 114.871981) (end 139.16742 114.499222) (width 0.2) (layer "F.Cu") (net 5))
 (segment (start 137.075 115.5) (end 137.235513 115.5) (width 0.2) (layer "F.Cu") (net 5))
 (segment (start 135.795576 112.795576) (end 136.890531 112.795576) (width 0.2) (layer "F.Cu") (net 5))
 (segment (start 138.053019 114.871981) (end 138.794661 114.871981) (width 0.2) (layer "F.Cu") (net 5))
 (via (at 142.5 115.104588) (size 0.4) (drill 0.2) (layers "F.Cu" "B.Cu") (free yes) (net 5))
 (via (at 135.5 114.85) (size 0.4) (drill 0.2) (layers "F.Cu" "B.Cu") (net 5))
 (via (at 137.753005 116.599061) (size 0.4) (drill 0.2) (layers "F.Cu" "B.Cu") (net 5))
 (segment (start 137.454178 116.599061) (end 137.44734 116.605899) (width 0.07) (layer "B.Cu") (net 5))
 (segment (start 135.338656 115.011344) (end 135.5 114.85) (width 0.07) (layer "B.Cu") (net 5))
 (segment (start 138.584629 116.486084) (end 139.171713 115.899) (width 0.2) (layer "B.Cu") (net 5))
 (segment (start 135.882597 116.5) (end 135.338656 115.956059) (width 0.07) (layer "B.Cu") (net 5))
 (segment (start 137.865982 116.486084) (end 137.753005 116.599061) (width 0.2) (layer "B.Cu") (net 5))
 (segment (start 139.171713 115.899) (end 141.899 115.899) (width 0.2) (layer "B.Cu") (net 5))
 (segment (start 137.021667 116.5) (end 135.882597 116.5) (width 0.07) (layer "B.Cu") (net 5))
 (segment (start 142.5 115.851905) (end 144.204268 115.851905) (width 0.2) (layer "B.Cu") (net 5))
 (segment (start 137.127566 116.605899) (end 137.021667 116.5) (width 0.07) (layer "B.Cu") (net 5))
 (segment (start 137.44734 116.605899) (end 137.127566 116.605899) (width 0.07) (layer "B.Cu") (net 5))
 (segment (start 141.899 115.899) (end 141.946095 115.851905) (width 0.2) (layer "B.Cu") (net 5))
 (segment (start 142.5 115.851905) (end 142.5 115.104588) (width 0.07) (layer "B.Cu") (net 5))
 (segment (start 138.584629 116.486084) (end 137.865982 116.486084) (width 0.2) (layer "B.Cu") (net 5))
 (segment (start 137.753005 116.599061) (end 137.454178 116.599061) (width 0.07) (layer "B.Cu") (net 5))
 (segment (start 141.946095 115.851905) (end 142.5 115.851905) (width 0.2) (layer "B.Cu") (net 5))
 (segment (start 135.338656 115.956059) (end 135.338656 115.011344) (width 0.07) (layer "B.Cu") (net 5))
 (segment (start 137.375 114.75) (end 137.75 114.75) (width 0.07) (layer "F.Cu") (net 6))
 (segment (start 137.75 114.75) (end 138.000778 114.499222) (width 0.07) (layer "F.Cu") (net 6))
 (segment (start 138.000778 114.499222) (end 138.36742 114.499222) (width 0.07) (layer "F.Cu") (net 6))
 (segment (start 133.95 114.45) (end 134.89565 115.39565) (width 0.2) (layer "F.Cu") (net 10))
 (segment (start 132 114.45) (end 133.95 114.45) (width 0.2) (layer "F.Cu") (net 10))
 (segment (start 136.07935 115.39565) (end 134.89565 115.39565) (width 0.07) (layer "F.Cu") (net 10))
 (segment (start 136.475 115) (end 136.07935 115.39565) (width 0.07) (layer "F.Cu") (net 10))
 (segment (start 138.021 113.479) (end 138.979 113.479) (width 0.1) (layer "F.Cu") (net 7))
 (segment (start 137.675 114.5) (end 137.932124 114.242876) (width 0.1) (layer "F.Cu") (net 7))
 (segment (start 138.979 113.479) (end 139.3 113.8) (width 0.1) (layer "F.Cu") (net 7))
 (segment (start 137.932124 113.567876) (end 138.021 113.479) (width 0.1) (layer "F.Cu") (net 7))
 (segment (start 137.932124 114.242876) (end 137.932124 113.567876) (width 0.1) (layer "F.Cu") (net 7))
 (segment (start 143.3998 115.500001) (end 140.530174 115.500001) (width 0.07) (layer "F.Cu") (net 4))
 (segment (start 143.973063 116.314755) (end 143.814755 116.314755) (width 0.07) (layer "F.Cu") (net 4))
 (segment (start 135.494 115.994) (end 135.559 116.059) (width 0.07) (layer "F.Cu") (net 4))
 (segment (start 135.006 115.994) (end 135.494 115.994) (width 0.07) (layer "F.Cu") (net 4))
 (segment (start 134.45 115.45) (end 132 115.45) (width 0.2) (layer "F.Cu") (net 4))
 (segment (start 140.530174 115.500001) (end 140.309284 115.279111) (width 0.07) (layer "F.Cu") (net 4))
 (segment (start 143.3998 115.8998) (end 143.3998 115.500001) (width 0.07) (layer "F.Cu") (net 4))
 (segment (start 136.178828 115.796172) (end 135.724656 115.796172) (width 0.07) (layer "F.Cu") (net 4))
 (segment (start 135 116) (end 135.006 115.994) (width 0.07) (layer "F.Cu") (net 4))
 (segment (start 135.916 116.059) (end 136.475 115.5) (width 0.07) (layer "F.Cu") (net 4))
 (segment (start 135.559 116.059) (end 135.916 116.059) (width 0.07) (layer "F.Cu") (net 4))
 (segment (start 143.814755 116.314755) (end 143.3998 115.8998) (width 0.07) (layer "F.Cu") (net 4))
 (segment (start 135 116) (end 134.45 115.45) (width 0.2) (layer "F.Cu") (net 4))
 (segment (start 136.475 115.5) (end 136.178828 115.796172) (width 0.07) (layer "F.Cu") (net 4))
 (via (at 140.309284 115.279111) (size 0.4) (drill 0.2) (layers "F.Cu" "B.Cu") (free yes) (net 4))
 (via (at 135.724656 115.796172) (size 0.4) (drill 0.2) (layers "F.Cu" "B.Cu") (free yes) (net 4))
 (segment (start 135.724656 115.796172) (end 135.781061 115.739767) (width 0.07) (layer "B.Cu") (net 4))
 (segment (start 138.739768 115.513654) (end 138.739768 115.5) (width 0.07) (layer "B.Cu") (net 4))
 (segment (start 138.513655 115.739767) (end 138.739768 115.513654) (width 0.07) (layer "B.Cu") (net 4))
 (segment (start 135.781061 115.739767) (end 138.513655 115.739767) (width 0.07) (layer "B.Cu") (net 4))
 (segment (start 140.088395 115.5) (end 140.309284 115.279111) (width 0.07) (layer "B.Cu") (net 4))
 (segment (start 138.739768 115.5) (end 140.088395 115.5) (width 0.07) (layer "B.Cu") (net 4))
 (segment (start 135.784887 115.236) (end 135.340113 115.236) (width 0.07) (layer "F.Cu") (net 11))
 (segment (start 136.7435 114.7815) (end 136.775 114.75) (width 0.07) (layer "F.Cu") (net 11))
 (segment (start 136.270887 114.75) (end 135.802887 115.218) (width 0.07) (layer "F.Cu") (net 11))
 (segment (start 134.912798 114.808685) (end 134.912798 114.087202) (width 0.2) (layer "F.Cu") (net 11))
 (segment (start 135.802887 115.218) (end 135.784887 115.236) (width 0.07) (layer "F.Cu") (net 11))
 (segment (start 136.775 114.75) (end 136.297738 114.75) (width 0.07) (layer "F.Cu") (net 11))
 (segment (start 135.340113 115.236) (end 134.912798 114.808685) (width 0.07) (layer "F.Cu") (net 11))
 (segment (start 134.275596 113.45) (end 132 113.45) (width 0.2) (layer "F.Cu") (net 11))
 (segment (start 134.912798 114.087202) (end 134.275596 113.45) (width 0.2) (layer "F.Cu") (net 11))
 (segment (start 136.297738 114.75) (end 136.270887 114.75) (width 0.07) (layer "F.Cu") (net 11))
 (segment (start 133.766152 112.45) (end 132 112.45) (width 0.2) (layer "F.Cu") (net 8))
 (segment (start 134.892696 113.576544) (end 135.485152 114.169) (width 0.07) (layer "F.Cu") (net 8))
 (segment (start 134.892696 113.576544) (end 133.766152 112.45) (width 0.2) (layer "F.Cu") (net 8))
 (segment (start 135.579353 114.169) (end 135.878494 114.468141) (width 0.07) (layer "F.Cu") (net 8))
 (segment (start 135.485152 114.169) (end 135.579353 114.169) (width 0.07) (layer "F.Cu") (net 8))
 (segment (start 135.962912 114.5) (end 136.475 114.5) (width 0.07) (layer "F.Cu") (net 8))
 (segment (start 135.808933 114.090138) (end 135.248706 113.529911) (width 0.07) (layer "F.Cu") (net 12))
 (segment (start 135.808933 114.092435) (end 135.808933 114.090138) (width 0.07) (layer "F.Cu") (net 12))
 (segment (start 135.966498 114.25) (end 135.808933 114.092435) (width 0.07) (layer "F.Cu") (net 12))
 (segment (start 135.248706 113.529911) (end 135.248706 113.006706) (width 0.2) (layer "F.Cu") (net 12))
 (segment (start 136.775 114.25) (end 135.966498 114.25) (width 0.07) (layer "F.Cu") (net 12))
 (segment (start 135.248706 113.006706) (end 133.692 111.45) (width 0.2) (layer "F.Cu") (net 12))
 (segment (start 133.692 111.45) (end 132 111.45) (width 0.2) (layer "F.Cu") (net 12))
 (segment (start 142.764427 114.010614) (end 143.389185 114.010614) (width 0.07) (layer "F.Cu") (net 2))
 (segment (start 142.764427 114.010614) (end 143.579207 113.195834) (width 0.07) (layer "F.Cu") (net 2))
 (segment (start 134.95 116.45) (end 132 116.45) (width 0.2) (layer "F.Cu") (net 2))
 (segment (start 143.389185 114.010614) (end 143.3998 113.999999) (width 0.07) (layer "F.Cu") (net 2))
 (segment (start 136.775 115.25) (end 136.775 116) (width 0.07) (layer "F.Cu") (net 2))
 (segment (start 136.694899 116.219899) (end 136.675 116.2) (width 0.07) (layer "F.Cu") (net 2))
 (segment (start 135.225 116.2) (end 134.975 116.45) (width 0.2) (layer "F.Cu") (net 2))
 (segment (start 143.579207 113.195834) (end 143.995667 113.195834) (width 0.07) (layer "F.Cu") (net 2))
 (segment (start 135.325 116.2) (end 135.225 116.2) (width 0.2) (layer "F.Cu") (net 2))
 (segment (start 136.775 116) (end 136.675 116.1) (width 0.07) (layer "F.Cu") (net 2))
 (segment (start 135.325 116.2) (end 136.675 116.2) (width 0.07) (layer "F.Cu") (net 2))
 (segment (start 137.287453 116.219899) (end 136.694899 116.219899) (width 0.07) (layer "F.Cu") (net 2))
 (segment (start 132.25 116.2) (end 132 116.45) (width 0.07) (layer "F.Cu") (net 2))
 (via (at 137.287453 116.219899) (size 0.4) (drill 0.2) (layers "F.Cu" "B.Cu") (free yes) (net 2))
 (via (at 142.764427 114.010614) (size 0.4) (drill 0.2) (layers "F.Cu" "B.Cu") (free yes) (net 2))
 (segment (start 142.497241 114.502759) (end 142.497241 114.490834) (width 0.07) (layer "B.Cu") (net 2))
 (segment (start 137.582303 115.925049) (end 138.854336 115.925049) (width 0.07) (layer "B.Cu") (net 2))
 (segment (start 141.332224 115.667776) (end 142.497241 114.502759) (width 0.07) (layer "B.Cu") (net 2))
 (segment (start 139.111609 115.667776) (end 141.332224 115.667776) (width 0.07) (layer "B.Cu") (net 2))
 (segment (start 137.287453 116.219899) (end 137.582303 115.925049) (width 0.07) (layer "B.Cu") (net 2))
 (segment (start 142.5 114.488075) (end 142.5 114.275041) (width 0.07) (layer "B.Cu") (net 2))
 (segment (start 138.854336 115.925049) (end 139.111609 115.667776) (width 0.07) (layer "B.Cu") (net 2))
 (segment (start 142.5 114.275041) (end 142.764427 114.010614) (width 0.07) (layer "B.Cu") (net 2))
 (segment (start 142.497241 114.490834) (end 142.5 114.488075) (width 0.07) (layer "B.Cu") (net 2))
 (segment (start 138.307436 115.989634) (end 138.305223 115.987421) (width 0.2) (layer "F.Cu") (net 9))
 (segment (start 140.060827 117.279506) (end 140.060827 116.477122) (width 0.2) (layer "F.Cu") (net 9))
 (segment (start 139.579016 115.989634) (end 138.307436 115.989634) (width 0.2) (layer "F.Cu") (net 9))
 (segment (start 139.554152 117.762208) (end 107.440827 117.762208) (width 0.2) (layer "F.Cu") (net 9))
 (segment (start 140.060827 116.477122) (end 140.061623 116.476326) (width 0.2) (layer "F.Cu") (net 9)))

